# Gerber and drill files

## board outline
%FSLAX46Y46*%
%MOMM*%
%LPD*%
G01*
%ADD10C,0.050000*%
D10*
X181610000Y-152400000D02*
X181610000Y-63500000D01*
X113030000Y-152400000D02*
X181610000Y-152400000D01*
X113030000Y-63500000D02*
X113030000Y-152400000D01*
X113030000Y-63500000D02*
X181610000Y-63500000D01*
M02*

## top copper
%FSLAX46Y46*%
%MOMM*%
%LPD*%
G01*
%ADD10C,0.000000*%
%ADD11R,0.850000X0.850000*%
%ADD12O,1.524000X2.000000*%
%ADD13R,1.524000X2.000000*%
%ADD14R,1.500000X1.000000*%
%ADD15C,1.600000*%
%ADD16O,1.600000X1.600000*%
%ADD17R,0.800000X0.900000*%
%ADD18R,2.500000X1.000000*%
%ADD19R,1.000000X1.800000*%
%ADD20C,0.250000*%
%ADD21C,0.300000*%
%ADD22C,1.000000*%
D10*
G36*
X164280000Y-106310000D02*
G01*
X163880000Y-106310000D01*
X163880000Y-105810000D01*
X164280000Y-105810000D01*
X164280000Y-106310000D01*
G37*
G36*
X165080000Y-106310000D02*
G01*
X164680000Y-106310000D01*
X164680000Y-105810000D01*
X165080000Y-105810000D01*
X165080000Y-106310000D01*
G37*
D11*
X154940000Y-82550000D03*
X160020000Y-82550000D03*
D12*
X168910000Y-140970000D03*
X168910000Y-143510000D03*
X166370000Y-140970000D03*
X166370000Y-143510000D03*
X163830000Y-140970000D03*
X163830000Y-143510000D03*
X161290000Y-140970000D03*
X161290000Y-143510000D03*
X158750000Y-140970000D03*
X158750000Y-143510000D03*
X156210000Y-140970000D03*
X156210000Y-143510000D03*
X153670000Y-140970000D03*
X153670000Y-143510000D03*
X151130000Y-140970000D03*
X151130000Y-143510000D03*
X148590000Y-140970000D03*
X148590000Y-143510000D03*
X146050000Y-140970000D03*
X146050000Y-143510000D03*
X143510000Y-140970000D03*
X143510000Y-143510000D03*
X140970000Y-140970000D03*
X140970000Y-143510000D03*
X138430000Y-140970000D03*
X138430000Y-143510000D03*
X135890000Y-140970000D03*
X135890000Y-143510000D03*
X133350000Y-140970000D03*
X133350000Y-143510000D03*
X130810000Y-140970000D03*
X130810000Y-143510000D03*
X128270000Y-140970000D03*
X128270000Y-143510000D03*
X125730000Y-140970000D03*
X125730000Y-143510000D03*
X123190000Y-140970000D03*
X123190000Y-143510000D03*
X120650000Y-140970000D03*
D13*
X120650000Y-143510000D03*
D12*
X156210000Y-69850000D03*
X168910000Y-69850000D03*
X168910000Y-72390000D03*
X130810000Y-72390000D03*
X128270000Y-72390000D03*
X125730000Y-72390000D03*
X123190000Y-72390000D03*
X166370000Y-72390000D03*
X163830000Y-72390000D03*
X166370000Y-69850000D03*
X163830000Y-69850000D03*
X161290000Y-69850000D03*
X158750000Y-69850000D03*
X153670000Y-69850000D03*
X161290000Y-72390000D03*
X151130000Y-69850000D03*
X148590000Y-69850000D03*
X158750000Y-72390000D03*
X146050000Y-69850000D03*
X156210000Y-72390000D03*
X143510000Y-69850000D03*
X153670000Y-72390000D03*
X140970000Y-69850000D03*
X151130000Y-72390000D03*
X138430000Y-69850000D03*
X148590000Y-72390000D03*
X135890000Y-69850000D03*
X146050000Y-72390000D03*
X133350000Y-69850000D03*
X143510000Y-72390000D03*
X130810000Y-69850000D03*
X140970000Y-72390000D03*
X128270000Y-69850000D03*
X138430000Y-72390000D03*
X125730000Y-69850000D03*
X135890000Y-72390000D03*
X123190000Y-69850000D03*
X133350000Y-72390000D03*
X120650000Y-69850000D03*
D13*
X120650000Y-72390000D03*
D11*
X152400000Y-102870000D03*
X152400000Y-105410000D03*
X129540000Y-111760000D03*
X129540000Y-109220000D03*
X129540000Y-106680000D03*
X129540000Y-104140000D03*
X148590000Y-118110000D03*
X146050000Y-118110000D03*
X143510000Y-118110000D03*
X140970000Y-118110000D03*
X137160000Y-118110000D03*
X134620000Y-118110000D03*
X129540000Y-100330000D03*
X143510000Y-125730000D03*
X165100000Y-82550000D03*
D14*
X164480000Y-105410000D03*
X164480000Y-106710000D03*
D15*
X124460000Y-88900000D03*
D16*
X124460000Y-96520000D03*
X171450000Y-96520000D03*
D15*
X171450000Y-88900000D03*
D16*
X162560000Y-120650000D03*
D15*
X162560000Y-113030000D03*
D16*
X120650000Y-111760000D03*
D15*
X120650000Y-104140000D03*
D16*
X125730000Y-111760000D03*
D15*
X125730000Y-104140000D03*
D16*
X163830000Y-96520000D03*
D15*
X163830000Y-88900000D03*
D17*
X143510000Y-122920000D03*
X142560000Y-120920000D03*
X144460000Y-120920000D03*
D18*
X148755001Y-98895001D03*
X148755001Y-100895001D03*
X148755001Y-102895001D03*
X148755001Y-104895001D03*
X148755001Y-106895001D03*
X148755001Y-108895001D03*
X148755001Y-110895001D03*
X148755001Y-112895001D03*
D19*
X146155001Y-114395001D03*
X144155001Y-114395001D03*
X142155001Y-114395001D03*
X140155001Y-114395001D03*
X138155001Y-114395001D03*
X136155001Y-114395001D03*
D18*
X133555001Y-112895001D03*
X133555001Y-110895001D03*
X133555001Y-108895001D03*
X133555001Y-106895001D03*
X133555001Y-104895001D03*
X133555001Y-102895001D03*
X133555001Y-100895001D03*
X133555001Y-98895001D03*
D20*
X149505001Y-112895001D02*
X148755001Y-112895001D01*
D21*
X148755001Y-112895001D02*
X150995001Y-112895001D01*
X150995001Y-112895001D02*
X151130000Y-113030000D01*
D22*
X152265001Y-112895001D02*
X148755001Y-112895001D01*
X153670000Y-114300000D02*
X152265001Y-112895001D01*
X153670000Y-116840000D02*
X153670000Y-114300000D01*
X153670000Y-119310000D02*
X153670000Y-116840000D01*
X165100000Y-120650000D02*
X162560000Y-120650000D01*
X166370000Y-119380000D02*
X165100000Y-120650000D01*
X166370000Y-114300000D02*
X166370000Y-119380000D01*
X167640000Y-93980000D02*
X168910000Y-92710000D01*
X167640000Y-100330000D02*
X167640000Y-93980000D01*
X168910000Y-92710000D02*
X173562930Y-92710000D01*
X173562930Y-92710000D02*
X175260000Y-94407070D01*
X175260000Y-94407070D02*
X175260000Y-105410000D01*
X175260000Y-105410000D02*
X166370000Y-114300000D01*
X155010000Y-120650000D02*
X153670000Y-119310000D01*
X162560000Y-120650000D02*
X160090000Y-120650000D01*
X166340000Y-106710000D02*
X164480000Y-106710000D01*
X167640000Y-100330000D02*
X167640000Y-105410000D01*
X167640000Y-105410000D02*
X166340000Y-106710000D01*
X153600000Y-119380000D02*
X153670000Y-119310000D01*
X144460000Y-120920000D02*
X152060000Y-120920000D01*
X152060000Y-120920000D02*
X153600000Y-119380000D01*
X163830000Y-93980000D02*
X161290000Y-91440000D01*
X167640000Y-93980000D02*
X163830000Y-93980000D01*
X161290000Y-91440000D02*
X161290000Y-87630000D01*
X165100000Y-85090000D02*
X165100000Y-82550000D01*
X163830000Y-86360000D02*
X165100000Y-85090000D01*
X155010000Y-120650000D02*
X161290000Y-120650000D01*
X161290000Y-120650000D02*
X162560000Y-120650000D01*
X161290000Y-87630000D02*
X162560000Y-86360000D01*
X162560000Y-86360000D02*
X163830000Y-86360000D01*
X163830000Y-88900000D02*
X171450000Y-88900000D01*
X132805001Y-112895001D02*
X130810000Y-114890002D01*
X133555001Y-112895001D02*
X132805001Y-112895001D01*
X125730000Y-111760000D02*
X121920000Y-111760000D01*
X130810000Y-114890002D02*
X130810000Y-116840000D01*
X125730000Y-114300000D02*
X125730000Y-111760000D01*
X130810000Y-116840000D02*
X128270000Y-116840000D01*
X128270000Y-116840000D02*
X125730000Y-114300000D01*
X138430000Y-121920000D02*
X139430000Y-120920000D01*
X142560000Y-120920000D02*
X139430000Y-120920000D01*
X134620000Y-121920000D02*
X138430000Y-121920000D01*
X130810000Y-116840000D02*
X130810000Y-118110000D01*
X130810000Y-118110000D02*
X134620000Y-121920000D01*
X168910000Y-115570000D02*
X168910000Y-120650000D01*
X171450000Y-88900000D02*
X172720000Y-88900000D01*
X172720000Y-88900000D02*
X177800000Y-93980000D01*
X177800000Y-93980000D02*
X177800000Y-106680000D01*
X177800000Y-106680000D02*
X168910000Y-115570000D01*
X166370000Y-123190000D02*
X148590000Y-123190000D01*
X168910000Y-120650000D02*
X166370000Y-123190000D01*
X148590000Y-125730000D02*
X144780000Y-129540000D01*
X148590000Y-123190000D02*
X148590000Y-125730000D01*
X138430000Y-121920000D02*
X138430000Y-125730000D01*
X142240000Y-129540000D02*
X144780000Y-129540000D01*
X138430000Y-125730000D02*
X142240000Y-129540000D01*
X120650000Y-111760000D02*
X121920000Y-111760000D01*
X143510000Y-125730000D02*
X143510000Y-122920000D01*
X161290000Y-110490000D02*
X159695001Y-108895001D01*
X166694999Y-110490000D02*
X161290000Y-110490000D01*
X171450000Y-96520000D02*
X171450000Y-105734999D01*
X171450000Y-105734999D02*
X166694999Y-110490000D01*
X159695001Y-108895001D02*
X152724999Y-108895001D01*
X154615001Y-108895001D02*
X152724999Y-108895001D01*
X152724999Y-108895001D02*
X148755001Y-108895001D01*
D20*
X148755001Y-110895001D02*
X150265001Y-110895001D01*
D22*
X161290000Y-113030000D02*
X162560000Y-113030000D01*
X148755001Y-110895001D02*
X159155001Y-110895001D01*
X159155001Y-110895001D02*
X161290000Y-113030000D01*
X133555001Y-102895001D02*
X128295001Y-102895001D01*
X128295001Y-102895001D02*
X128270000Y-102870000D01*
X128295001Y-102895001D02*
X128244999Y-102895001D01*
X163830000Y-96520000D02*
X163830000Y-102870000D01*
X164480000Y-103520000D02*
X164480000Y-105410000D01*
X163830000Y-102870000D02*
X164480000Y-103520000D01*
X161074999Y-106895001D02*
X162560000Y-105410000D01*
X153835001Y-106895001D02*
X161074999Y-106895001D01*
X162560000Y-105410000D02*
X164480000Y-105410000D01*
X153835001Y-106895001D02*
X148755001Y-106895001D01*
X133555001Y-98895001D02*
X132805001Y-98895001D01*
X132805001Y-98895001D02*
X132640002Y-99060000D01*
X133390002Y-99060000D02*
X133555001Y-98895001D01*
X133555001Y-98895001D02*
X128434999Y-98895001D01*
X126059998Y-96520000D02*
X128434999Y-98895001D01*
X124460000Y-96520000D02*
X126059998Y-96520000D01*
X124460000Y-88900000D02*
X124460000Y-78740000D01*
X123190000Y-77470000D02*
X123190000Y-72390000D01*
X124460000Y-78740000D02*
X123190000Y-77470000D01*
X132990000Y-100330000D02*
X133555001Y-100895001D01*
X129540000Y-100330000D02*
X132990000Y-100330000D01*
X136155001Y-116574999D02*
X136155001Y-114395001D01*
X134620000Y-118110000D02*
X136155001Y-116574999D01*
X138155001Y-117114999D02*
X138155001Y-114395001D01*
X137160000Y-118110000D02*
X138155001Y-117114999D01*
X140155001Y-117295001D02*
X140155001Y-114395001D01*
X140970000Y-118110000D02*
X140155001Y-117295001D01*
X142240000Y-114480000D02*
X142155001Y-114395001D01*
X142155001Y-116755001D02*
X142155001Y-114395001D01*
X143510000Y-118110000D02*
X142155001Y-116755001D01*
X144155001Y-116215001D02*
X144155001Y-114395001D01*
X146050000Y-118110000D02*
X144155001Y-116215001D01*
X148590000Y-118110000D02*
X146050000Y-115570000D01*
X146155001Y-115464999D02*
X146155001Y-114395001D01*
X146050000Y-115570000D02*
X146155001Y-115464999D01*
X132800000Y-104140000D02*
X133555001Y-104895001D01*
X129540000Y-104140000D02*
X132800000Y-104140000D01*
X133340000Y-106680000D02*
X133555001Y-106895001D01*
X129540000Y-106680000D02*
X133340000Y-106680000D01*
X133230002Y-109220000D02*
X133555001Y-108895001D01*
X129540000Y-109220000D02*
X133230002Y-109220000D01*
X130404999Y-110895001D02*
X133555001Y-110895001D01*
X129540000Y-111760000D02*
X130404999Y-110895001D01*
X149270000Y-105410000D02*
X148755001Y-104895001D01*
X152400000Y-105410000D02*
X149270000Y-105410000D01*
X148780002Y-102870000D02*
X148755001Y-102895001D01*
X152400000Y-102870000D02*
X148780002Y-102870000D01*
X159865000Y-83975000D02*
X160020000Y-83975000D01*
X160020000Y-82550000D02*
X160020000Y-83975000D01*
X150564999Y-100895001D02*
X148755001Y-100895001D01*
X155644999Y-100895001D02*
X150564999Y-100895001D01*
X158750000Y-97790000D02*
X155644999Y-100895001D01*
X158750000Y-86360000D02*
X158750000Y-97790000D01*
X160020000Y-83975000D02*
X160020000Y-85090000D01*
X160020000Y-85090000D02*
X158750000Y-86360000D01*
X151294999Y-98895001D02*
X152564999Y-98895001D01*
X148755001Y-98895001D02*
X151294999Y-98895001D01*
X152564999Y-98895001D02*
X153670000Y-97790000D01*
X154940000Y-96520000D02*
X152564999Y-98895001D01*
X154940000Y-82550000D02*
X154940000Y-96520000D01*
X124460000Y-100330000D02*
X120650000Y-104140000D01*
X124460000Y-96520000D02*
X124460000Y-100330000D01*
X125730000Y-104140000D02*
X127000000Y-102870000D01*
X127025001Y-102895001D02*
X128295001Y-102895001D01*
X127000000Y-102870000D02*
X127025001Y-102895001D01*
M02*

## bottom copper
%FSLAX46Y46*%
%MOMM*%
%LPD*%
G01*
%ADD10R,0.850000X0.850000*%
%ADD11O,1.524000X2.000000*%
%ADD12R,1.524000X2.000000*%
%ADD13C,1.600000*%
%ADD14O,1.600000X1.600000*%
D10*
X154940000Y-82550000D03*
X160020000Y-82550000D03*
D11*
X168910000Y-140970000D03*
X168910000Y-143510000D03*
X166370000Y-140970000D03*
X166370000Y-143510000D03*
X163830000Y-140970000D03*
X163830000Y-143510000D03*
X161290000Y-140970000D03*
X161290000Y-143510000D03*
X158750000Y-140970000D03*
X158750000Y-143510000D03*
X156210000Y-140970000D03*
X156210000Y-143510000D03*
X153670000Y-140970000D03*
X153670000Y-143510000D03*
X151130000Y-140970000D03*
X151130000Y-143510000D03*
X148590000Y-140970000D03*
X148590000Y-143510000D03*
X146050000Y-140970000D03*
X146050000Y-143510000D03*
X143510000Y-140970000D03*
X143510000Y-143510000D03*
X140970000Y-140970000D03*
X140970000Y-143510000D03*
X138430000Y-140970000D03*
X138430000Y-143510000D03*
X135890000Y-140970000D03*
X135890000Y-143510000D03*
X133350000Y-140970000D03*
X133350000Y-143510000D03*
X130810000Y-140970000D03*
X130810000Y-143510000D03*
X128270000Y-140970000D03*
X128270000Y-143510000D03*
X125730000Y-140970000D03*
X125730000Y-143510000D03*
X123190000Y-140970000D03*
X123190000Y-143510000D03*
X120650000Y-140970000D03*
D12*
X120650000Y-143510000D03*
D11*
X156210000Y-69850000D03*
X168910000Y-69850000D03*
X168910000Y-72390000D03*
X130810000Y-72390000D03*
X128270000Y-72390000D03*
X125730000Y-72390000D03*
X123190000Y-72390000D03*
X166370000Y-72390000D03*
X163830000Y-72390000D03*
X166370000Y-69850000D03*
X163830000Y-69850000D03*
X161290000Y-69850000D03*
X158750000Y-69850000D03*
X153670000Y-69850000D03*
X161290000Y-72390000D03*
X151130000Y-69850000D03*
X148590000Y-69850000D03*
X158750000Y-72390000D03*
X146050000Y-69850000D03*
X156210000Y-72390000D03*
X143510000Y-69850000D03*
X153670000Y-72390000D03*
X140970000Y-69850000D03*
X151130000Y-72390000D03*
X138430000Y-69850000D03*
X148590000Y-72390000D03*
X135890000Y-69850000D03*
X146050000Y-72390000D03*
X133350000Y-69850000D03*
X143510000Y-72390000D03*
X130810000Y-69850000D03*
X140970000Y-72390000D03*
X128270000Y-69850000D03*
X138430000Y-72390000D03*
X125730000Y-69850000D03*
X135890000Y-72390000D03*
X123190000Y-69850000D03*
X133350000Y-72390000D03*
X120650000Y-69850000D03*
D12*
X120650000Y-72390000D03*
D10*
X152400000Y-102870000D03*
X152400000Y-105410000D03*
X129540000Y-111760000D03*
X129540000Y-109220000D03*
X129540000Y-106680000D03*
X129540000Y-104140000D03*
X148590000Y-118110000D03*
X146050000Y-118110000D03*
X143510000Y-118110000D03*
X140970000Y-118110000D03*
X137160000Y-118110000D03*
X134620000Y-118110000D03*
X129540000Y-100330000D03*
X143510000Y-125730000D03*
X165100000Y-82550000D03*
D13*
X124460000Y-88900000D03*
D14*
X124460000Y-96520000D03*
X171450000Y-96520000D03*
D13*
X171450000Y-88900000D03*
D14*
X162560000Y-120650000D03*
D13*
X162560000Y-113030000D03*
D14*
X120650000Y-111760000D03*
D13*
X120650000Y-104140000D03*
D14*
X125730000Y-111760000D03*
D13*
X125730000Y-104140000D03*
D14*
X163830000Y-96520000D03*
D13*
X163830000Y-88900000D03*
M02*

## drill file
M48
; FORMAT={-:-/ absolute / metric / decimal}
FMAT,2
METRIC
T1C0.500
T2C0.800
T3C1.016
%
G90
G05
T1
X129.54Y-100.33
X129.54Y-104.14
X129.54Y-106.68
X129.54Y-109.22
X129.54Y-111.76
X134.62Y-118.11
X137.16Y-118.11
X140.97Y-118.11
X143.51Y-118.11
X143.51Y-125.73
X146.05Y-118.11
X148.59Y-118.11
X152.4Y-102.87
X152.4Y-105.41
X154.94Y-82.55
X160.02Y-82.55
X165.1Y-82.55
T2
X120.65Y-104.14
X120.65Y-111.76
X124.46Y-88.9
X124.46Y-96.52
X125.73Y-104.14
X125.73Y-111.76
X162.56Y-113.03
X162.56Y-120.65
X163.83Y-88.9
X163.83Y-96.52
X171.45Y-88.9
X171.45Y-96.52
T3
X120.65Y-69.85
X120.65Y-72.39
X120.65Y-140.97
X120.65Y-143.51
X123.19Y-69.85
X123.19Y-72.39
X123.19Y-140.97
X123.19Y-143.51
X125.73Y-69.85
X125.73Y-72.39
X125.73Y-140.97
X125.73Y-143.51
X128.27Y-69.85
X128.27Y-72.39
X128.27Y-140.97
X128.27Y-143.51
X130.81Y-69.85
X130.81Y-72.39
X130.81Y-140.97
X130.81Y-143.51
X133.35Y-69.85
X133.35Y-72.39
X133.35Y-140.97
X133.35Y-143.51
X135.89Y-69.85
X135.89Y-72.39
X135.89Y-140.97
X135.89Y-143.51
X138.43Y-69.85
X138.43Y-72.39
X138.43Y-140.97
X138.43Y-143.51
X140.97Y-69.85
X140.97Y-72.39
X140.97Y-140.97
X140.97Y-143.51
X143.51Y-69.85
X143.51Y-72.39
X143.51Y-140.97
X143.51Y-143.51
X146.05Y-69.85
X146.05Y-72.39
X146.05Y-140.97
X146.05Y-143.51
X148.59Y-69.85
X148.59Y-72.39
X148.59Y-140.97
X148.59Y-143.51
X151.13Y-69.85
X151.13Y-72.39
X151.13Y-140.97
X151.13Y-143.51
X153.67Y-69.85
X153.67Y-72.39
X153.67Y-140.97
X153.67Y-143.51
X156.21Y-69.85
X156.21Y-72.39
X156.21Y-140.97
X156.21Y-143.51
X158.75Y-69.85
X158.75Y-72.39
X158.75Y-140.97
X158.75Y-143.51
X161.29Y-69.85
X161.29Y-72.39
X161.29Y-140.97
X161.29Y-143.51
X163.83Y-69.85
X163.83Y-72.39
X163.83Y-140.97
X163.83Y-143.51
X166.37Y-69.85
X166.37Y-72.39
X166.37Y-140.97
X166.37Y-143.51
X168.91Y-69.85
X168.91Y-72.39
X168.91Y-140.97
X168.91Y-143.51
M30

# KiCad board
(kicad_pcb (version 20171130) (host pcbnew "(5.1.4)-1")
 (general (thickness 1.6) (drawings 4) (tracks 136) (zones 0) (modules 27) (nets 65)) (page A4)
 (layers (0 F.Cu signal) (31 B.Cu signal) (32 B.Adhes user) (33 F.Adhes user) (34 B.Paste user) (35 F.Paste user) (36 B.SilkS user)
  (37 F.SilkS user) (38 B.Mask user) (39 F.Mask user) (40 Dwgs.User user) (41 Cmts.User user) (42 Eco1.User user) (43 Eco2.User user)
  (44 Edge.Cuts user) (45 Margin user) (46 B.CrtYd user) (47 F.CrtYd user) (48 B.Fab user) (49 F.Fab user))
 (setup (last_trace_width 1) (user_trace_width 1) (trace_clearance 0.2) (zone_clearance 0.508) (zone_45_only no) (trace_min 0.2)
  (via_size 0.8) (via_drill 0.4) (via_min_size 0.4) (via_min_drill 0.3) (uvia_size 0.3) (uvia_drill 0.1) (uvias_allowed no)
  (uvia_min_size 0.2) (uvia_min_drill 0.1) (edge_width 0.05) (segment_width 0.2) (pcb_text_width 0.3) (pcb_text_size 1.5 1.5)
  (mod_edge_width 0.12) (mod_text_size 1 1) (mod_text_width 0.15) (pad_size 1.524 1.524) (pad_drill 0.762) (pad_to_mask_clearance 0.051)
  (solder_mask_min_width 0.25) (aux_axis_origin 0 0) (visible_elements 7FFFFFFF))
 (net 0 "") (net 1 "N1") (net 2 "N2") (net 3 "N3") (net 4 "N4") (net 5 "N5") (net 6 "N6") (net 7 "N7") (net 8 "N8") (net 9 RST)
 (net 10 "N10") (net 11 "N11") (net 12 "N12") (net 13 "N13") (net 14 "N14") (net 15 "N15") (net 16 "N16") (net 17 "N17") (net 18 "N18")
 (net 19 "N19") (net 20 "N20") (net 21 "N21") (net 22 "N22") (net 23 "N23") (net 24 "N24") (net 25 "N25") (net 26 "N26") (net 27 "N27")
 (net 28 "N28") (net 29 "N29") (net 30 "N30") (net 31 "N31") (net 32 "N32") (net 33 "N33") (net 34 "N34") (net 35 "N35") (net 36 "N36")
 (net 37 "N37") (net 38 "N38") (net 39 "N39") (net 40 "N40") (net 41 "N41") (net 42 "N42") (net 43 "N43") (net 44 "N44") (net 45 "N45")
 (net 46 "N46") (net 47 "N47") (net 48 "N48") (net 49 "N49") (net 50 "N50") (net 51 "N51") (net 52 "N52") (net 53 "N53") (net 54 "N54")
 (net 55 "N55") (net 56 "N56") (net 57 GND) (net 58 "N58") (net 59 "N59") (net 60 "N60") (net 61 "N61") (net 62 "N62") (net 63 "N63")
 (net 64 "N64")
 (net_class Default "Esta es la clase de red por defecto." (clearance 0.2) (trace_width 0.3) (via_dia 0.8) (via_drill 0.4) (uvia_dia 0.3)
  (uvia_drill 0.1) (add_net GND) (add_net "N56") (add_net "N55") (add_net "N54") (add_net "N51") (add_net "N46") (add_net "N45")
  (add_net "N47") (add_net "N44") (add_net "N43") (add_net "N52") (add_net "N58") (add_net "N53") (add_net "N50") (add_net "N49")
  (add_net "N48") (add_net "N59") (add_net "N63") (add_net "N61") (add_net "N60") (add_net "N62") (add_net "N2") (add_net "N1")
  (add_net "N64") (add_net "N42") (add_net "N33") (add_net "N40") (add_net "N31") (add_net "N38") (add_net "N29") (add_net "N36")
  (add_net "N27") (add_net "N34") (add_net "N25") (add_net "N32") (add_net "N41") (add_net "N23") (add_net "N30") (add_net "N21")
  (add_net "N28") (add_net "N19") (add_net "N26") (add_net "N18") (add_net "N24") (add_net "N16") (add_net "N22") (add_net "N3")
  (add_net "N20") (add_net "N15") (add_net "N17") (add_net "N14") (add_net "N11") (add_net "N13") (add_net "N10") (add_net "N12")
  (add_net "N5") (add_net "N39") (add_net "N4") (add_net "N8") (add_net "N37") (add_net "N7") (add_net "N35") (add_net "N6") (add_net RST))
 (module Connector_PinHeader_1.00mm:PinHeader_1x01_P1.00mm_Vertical (layer F.Cu) (at 154.94 82.55)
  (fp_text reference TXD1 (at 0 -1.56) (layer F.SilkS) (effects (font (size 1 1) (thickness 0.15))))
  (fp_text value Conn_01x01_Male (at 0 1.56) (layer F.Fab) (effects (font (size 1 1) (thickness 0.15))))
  (pad 1 thru_hole rect (at 0 0) (size 0.85 0.85) (drill 0.5) (layers *.Cu *.Mask) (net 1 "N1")))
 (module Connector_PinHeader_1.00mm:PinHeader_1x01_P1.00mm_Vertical (layer F.Cu) (at 160.02 82.55)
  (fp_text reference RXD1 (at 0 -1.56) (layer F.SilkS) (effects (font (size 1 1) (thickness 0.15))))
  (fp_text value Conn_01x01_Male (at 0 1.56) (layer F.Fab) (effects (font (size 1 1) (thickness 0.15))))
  (pad 1 thru_hole rect (at 0 0) (size 0.85 0.85) (drill 0.5) (layers *.Cu *.Mask) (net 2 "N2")))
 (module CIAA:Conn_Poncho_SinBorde (layer F.Cu) (at 120.65 72.39 90)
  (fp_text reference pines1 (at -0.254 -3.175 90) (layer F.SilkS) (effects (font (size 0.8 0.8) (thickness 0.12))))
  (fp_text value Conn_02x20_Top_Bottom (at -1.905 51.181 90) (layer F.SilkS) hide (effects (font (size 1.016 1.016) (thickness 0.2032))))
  (pad 80 thru_hole oval (at -68.58 48.26) (size 1.524 2) (drill 1.016) (layers *.Cu *.Mask F.SilkS))
  (pad 79 thru_hole oval (at -71.12 48.26) (size 1.524 2) (drill 1.016) (layers *.Cu *.Mask F.SilkS))
  (pad 78 thru_hole oval (at -68.58 45.72) (size 1.524 2) (drill 1.016) (layers *.Cu *.Mask F.SilkS))
  (pad 77 thru_hole oval (at -71.12 45.72) (size 1.524 2) (drill 1.016) (layers *.Cu *.Mask F.SilkS))
  (pad 76 thru_hole oval (at -68.58 43.18) (size 1.524 2) (drill 1.016) (layers *.Cu *.Mask F.SilkS))
  (pad 75 thru_hole oval (at -71.12 43.18) (size 1.524 2) (drill 1.016) (layers *.Cu *.Mask F.SilkS))
  (pad 74 thru_hole oval (at -68.58 40.64) (size 1.524 2) (drill 1.016) (layers *.Cu *.Mask F.SilkS))
  (pad 73 thru_hole oval (at -71.12 40.64) (size 1.524 2) (drill 1.016) (layers *.Cu *.Mask F.SilkS))
  (pad 72 thru_hole oval (at -68.58 38.1) (size 1.524 2) (drill 1.016) (layers *.Cu *.Mask F.SilkS))
  (pad 71 thru_hole oval (at -71.12 38.1) (size 1.524 2) (drill 1.016) (layers *.Cu *.Mask F.SilkS))
  (pad 70 thru_hole oval (at -68.58 35.56) (size 1.524 2) (drill 1.016) (layers *.Cu *.Mask F.SilkS))
  (pad 69 thru_hole oval (at -71.12 35.56) (size 1.524 2) (drill 1.016) (layers *.Cu *.Mask F.SilkS))
  (pad 68 thru_hole oval (at -68.58 33.02) (size 1.524 2) (drill 1.016) (layers *.Cu *.Mask F.SilkS))
  (pad 67 thru_hole oval (at -71.12 33.02) (size 1.524 2) (drill 1.016) (layers *.Cu *.Mask F.SilkS))
  (pad 66 thru_hole oval (at -68.58 30.48) (size 1.524 2) (drill 1.016) (layers *.Cu *.Mask F.SilkS))
  (pad 65 thru_hole oval (at -71.12 30.48) (size 1.524 2) (drill 1.016) (layers *.Cu *.Mask F.SilkS))
  (pad 64 thru_hole oval (at -68.58 27.94) (size 1.524 2) (drill 1.016) (layers *.Cu *.Mask F.SilkS))
  (pad 63 thru_hole oval (at -71.12 27.94) (size 1.524 2) (drill 1.016) (layers *.Cu *.Mask F.SilkS))
  (pad 62 thru_hole oval (at -68.58 25.4) (size 1.524 2) (drill 1.016) (layers *.Cu *.Mask F.SilkS))
  (pad 61 thru_hole oval (at -71.12 25.4) (size 1.524 2) (drill 1.016) (layers *.Cu *.Mask F.SilkS))
  (pad 60 thru_hole oval (at -68.58 22.86) (size 1.524 2) (drill 1.016) (layers *.Cu *.Mask F.SilkS))
  (pad 59 thru_hole oval (at -71.12 22.86) (size 1.524 2) (drill 1.016) (layers *.Cu *.Mask F.SilkS))
  (pad 58 thru_hole oval (at -68.58 20.32) (size 1.524 2) (drill 1.016) (layers *.Cu *.Mask F.SilkS))
  (pad 57 thru_hole oval (at -71.12 20.32) (size 1.524 2) (drill 1.016) (layers *.Cu *.Mask F.SilkS))
  (pad 56 thru_hole oval (at -68.58 17.78) (size 1.524 2) (drill 1.016) (layers *.Cu *.Mask F.SilkS))
  (pad 55 thru_hole oval (at -71.12 17.78) (size 1.524 2) (drill 1.016) (layers *.Cu *.Mask F.SilkS))
  (pad 54 thru_hole oval (at -68.58 15.24) (size 1.524 2) (drill 1.016) (layers *.Cu *.Mask F.SilkS))
  (pad 53 thru_hole oval (at -71.12 15.24) (size 1.524 2) (drill 1.016) (layers *.Cu *.Mask F.SilkS))
  (pad 52 thru_hole oval (at -68.58 12.7) (size 1.524 2) (drill 1.016) (layers *.Cu *.Mask F.SilkS))
  (pad 51 thru_hole oval (at -71.12 12.7) (size 1.524 2) (drill 1.016) (layers *.Cu *.Mask F.SilkS))
  (pad 50 thru_hole oval (at -68.58 10.16) (size 1.524 2) (drill 1.016) (layers *.Cu *.Mask F.SilkS))
  (pad 49 thru_hole oval (at -71.12 10.16) (size 1.524 2) (drill 1.016) (layers *.Cu *.Mask F.SilkS))
  (pad 48 thru_hole oval (at -68.58 7.62) (size 1.524 2) (drill 1.016) (layers *.Cu *.Mask F.SilkS))
  (pad 47 thru_hole oval (at -71.12 7.62) (size 1.524 2) (drill 1.016) (layers *.Cu *.Mask F.SilkS))
  (pad 46 thru_hole oval (at -68.58 5.08) (size 1.524 2) (drill 1.016) (layers *.Cu *.Mask F.SilkS))
  (pad 45 thru_hole oval (at -71.12 5.08) (size 1.524 2) (drill 1.016) (layers *.Cu *.Mask F.SilkS))
  (pad 44 thru_hole oval (at -68.58 2.54) (size 1.524 2) (drill 1.016) (layers *.Cu *.Mask F.SilkS))
  (pad 43 thru_hole oval (at -71.12 2.54) (size 1.524 2) (drill 1.016) (layers *.Cu *.Mask F.SilkS))
  (pad 42 thru_hole oval (at -68.58 0) (size 1.524 2) (drill 1.016) (layers *.Cu *.Mask F.SilkS))
  (pad 41 thru_hole rect (at -71.12 0) (size 1.524 2) (drill 1.016) (layers *.Cu *.Mask F.SilkS))
  (pad 30 thru_hole oval (at 2.54 35.56) (size 1.524 2) (drill 1.016) (layers *.Cu *.Mask F.SilkS) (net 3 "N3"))
  (pad 40 thru_hole oval (at 2.54 48.26) (size 1.524 2) (drill 1.016) (layers *.Cu *.Mask F.SilkS) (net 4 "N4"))
  (pad 39 thru_hole oval (at 0 48.26) (size 1.524 2) (drill 1.016) (layers *.Cu *.Mask F.SilkS) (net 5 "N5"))
  (pad 9 thru_hole oval (at 0 10.16) (size 1.524 2) (drill 1.016) (layers *.Cu *.Mask F.SilkS) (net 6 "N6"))
  (pad 7 thru_hole oval (at 0 7.62) (size 1.524 2) (drill 1.016) (layers *.Cu *.Mask F.SilkS) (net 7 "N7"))
  (pad 5 thru_hole oval (at 0 5.08) (size 1.524 2) (drill 1.016) (layers *.Cu *.Mask F.SilkS) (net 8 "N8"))
  (pad 3 thru_hole oval (at 0 2.54) (size 1.524 2) (drill 1.016) (layers *.Cu *.Mask F.SilkS) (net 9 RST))
  (pad 37 thru_hole oval (at 0 45.72) (size 1.524 2) (drill 1.016) (layers *.Cu *.Mask F.SilkS) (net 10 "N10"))
  (pad 35 thru_hole oval (at 0 43.18) (size 1.524 2) (drill 1.016) (layers *.Cu *.Mask F.SilkS) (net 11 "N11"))
  (pad 38 thru_hole oval (at 2.54 45.72) (size 1.524 2) (drill 1.016) (layers *.Cu *.Mask F.SilkS) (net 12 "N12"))
  (pad 36 thru_hole oval (at 2.54 43.18) (size 1.524 2) (drill 1.016) (layers *.Cu *.Mask F.SilkS) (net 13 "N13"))
  (pad 34 thru_hole oval (at 2.54 40.64) (size 1.524 2) (drill 1.016) (layers *.Cu *.Mask F.SilkS) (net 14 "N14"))
  (pad 32 thru_hole oval (at 2.54 38.1) (size 1.524 2) (drill 1.016) (layers *.Cu *.Mask F.SilkS) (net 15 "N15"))
  (pad 28 thru_hole oval (at 2.54 33.02) (size 1.524 2) (drill 1.016) (layers *.Cu *.Mask F.SilkS) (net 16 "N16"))
  (pad 33 thru_hole oval (at 0 40.64) (size 1.524 2) (drill 1.016) (layers *.Cu *.Mask F.SilkS) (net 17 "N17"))
  (pad 26 thru_hole oval (at 2.54 30.48) (size 1.524 2) (drill 1.016) (layers *.Cu *.Mask F.SilkS) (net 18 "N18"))
  (pad 24 thru_hole oval (at 2.54 27.94) (size 1.524 2) (drill 1.016) (layers *.Cu *.Mask F.SilkS) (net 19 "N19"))
  (pad 31 thru_hole oval (at 0 38.1) (size 1.524 2) (drill 1.016) (layers *.Cu *.Mask F.SilkS) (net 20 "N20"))
  (pad 22 thru_hole oval (at 2.54 25.4) (size 1.524 2) (drill 1.016) (layers *.Cu *.Mask F.SilkS) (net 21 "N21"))
  (pad 29 thru_hole oval (at 0 35.56) (size 1.524 2) (drill 1.016) (layers *.Cu *.Mask F.SilkS) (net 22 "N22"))
  (pad 20 thru_hole oval (at 2.54 22.86) (size 1.524 2) (drill 1.016) (layers *.Cu *.Mask F.SilkS) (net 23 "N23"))
  (pad 27 thru_hole oval (at 0 33.02) (size 1.524 2) (drill 1.016) (layers *.Cu *.Mask F.SilkS) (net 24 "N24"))
  (pad 18 thru_hole oval (at 2.54 20.32) (size 1.524 2) (drill 1.016) (layers *.Cu *.Mask F.SilkS) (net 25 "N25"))
  (pad 25 thru_hole oval (at 0 30.48) (size 1.524 2) (drill 1.016) (layers *.Cu *.Mask F.SilkS) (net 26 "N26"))
  (pad 16 thru_hole oval (at 2.54 17.78) (size 1.524 2) (drill 1.016) (layers *.Cu *.Mask F.SilkS) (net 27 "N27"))
  (pad 23 thru_hole oval (at 0 27.94) (size 1.524 2) (drill 1.016) (layers *.Cu *.Mask F.SilkS) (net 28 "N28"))
  (pad 14 thru_hole oval (at 2.54 15.24) (size 1.524 2) (drill 1.016) (layers *.Cu *.Mask F.SilkS) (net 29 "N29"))
  (pad 21 thru_hole oval (at 0 25.4) (size 1.524 2) (drill 1.016) (layers *.Cu *.Mask F.SilkS) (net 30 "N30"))
  (pad 12 thru_hole oval (at 2.54 12.7) (size 1.524 2) (drill 1.016) (layers *.Cu *.Mask F.SilkS) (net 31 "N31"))
  (pad 19 thru_hole oval (at 0 22.86) (size 1.524 2) (drill 1.016) (layers *.Cu *.Mask F.SilkS) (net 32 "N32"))
  (pad 10 thru_hole oval (at 2.54 10.16) (size 1.524 2) (drill 1.016) (layers *.Cu *.Mask F.SilkS) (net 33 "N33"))
  (pad 17 thru_hole oval (at 0 20.32) (size 1.524 2) (drill 1.016) (layers *.Cu *.Mask F.SilkS) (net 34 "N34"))
  (pad 8 thru_hole oval (at 2.54 7.62) (size 1.524 2) (drill 1.016) (layers *.Cu *.Mask F.SilkS) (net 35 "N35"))
  (pad 15 thru_hole oval (at 0 17.78) (size 1.524 2) (drill 1.016) (layers *.Cu *.Mask F.SilkS) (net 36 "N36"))
  (pad 6 thru_hole oval (at 2.54 5.08) (size 1.524 2) (drill 1.016) (layers *.Cu *.Mask F.SilkS) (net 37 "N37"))
  (pad 13 thru_hole oval (at 0 15.24) (size 1.524 2) (drill 1.016) (layers *.Cu *.Mask F.SilkS) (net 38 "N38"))
  (pad 4 thru_hole oval (at 2.54 2.54) (size 1.524 2) (drill 1.016) (layers *.Cu *.Mask F.SilkS) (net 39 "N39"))
  (pad 11 thru_hole oval (at 0 12.7) (size 1.524 2) (drill 1.016) (layers *.Cu *.Mask F.SilkS) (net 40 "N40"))
  (pad 2 thru_hole oval (at 2.54 0) (size 1.524 2) (drill 1.016) (layers *.Cu *.Mask F.SilkS) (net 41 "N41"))
  (pad 1 thru_hole rect (at 0 0) (size 1.524 2) (drill 1.016) (layers *.Cu *.Mask F.SilkS) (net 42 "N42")))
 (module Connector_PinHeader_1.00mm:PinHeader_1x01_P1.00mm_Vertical (layer F.Cu) (at 152.4 102.87)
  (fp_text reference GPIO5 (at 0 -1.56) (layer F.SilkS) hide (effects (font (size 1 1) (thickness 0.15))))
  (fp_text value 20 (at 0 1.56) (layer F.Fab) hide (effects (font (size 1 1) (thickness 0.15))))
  (pad 1 thru_hole rect (at 0 0) (size 0.85 0.85) (drill 0.5) (layers *.Cu *.Mask) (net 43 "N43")))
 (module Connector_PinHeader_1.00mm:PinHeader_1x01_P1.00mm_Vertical (layer F.Cu) (at 152.4 105.41)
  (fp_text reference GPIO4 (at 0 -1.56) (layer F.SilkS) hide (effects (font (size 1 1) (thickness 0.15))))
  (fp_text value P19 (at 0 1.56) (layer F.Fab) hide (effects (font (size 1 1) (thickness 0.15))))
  (pad 1 thru_hole rect (at 0 0) (size 0.85 0.85) (drill 0.5) (layers *.Cu *.Mask) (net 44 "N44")))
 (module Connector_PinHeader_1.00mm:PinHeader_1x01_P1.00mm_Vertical (layer F.Cu) (at 129.54 111.76)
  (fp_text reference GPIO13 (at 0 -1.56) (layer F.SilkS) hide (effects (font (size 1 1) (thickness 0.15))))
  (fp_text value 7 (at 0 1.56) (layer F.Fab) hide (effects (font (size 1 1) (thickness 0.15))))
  (pad 1 thru_hole rect (at 0 0) (size 0.85 0.85) (drill 0.5) (layers *.Cu *.Mask) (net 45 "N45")))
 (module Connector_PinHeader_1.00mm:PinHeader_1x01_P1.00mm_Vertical (layer F.Cu) (at 129.54 109.22)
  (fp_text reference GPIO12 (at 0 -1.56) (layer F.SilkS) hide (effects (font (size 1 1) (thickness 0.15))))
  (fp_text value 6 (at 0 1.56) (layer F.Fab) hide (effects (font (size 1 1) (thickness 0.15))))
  (pad 1 thru_hole rect (at 0 0) (size 0.85 0.85) (drill 0.5) (layers *.Cu *.Mask) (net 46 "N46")))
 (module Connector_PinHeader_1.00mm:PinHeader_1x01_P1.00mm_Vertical (layer F.Cu) (at 129.54 106.68)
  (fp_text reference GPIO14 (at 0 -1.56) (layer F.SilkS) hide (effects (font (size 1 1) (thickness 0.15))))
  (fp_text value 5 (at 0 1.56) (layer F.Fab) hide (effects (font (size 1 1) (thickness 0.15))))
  (pad 1 thru_hole rect (at 0 0) (size 0.85 0.85) (drill 0.5) (layers *.Cu *.Mask) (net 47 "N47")))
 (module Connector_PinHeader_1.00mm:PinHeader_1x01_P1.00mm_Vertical (layer F.Cu) (at 129.54 104.14)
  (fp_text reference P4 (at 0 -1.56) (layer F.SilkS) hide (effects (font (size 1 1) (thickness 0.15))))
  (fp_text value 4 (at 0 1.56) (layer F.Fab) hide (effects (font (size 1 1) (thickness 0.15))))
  (pad 1 thru_hole rect (at 0 0) (size 0.85 0.85) (drill 0.5) (layers *.Cu *.Mask) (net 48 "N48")))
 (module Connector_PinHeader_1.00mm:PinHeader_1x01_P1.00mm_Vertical (layer F.Cu) (at 148.59 118.11)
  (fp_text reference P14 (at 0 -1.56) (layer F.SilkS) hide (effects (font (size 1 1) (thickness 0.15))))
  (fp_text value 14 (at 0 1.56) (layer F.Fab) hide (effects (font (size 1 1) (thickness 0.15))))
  (pad 1 thru_hole rect (at 0 0) (size 0.85 0.85) (drill 0.5) (layers *.Cu *.Mask) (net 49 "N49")))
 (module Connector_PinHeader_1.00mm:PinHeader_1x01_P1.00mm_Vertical (layer F.Cu) (at 146.05 118.11)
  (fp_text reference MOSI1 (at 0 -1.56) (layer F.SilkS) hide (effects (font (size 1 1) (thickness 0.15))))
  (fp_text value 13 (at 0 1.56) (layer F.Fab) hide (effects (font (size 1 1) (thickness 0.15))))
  (pad 1 thru_hole rect (at 0 0) (size 0.85 0.85) (drill 0.5) (layers *.Cu *.Mask) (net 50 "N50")))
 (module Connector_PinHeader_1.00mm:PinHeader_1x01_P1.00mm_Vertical (layer F.Cu) (at 143.51 118.11)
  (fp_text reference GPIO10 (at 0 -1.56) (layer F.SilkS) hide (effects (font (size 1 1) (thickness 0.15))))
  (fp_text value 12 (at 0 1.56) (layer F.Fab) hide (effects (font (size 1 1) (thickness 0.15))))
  (pad 1 thru_hole rect (at 0 0) (size 0.85 0.85) (drill 0.5) (layers *.Cu *.Mask) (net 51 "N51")))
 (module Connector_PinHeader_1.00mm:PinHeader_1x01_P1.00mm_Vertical (layer F.Cu) (at 140.97 118.11)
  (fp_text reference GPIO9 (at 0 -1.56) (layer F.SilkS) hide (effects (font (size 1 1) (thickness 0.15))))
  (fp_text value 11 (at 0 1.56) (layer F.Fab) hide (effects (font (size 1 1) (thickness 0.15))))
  (pad 1 thru_hole rect (at 0 0) (size 0.85 0.85) (drill 0.5) (layers *.Cu *.Mask) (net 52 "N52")))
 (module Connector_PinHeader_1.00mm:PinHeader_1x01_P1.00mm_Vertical (layer F.Cu) (at 137.16 118.11)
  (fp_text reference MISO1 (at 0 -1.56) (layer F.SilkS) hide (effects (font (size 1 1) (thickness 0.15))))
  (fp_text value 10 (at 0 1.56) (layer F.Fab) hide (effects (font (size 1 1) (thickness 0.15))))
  (pad 1 thru_hole rect (at 0 0) (size 0.85 0.85) (drill 0.5) (layers *.Cu *.Mask) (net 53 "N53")))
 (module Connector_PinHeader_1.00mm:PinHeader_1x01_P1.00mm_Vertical (layer F.Cu) (at 134.62 118.11)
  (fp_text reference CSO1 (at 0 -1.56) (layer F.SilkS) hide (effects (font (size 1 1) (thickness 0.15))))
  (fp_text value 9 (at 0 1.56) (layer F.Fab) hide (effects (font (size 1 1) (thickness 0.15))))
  (pad 1 thru_hole rect (at 0 0) (size 0.85 0.85) (drill 0.5) (layers *.Cu *.Mask) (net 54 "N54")))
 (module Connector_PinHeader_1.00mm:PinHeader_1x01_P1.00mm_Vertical (layer F.Cu) (at 129.54 100.33)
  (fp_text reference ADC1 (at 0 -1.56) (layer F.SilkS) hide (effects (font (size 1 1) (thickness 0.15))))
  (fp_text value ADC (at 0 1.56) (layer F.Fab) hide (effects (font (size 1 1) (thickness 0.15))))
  (pad 1 thru_hole rect (at 0 0) (size 0.85 0.85) (drill 0.5) (layers *.Cu *.Mask) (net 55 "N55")))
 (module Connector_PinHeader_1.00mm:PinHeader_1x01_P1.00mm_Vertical (layer F.Cu) (at 143.51 125.73 180)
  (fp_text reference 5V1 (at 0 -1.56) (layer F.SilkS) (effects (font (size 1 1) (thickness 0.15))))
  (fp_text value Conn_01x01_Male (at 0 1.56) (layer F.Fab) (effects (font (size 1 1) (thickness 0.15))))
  (pad 1 thru_hole rect (at 0 0 180) (size 0.85 0.85) (drill 0.5) (layers *.Cu *.Mask) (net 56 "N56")))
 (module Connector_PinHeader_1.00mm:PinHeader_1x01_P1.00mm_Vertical (layer F.Cu) (at 165.1 82.55)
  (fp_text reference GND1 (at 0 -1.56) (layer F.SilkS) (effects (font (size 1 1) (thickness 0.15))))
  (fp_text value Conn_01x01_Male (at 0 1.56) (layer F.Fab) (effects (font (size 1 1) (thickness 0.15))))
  (pad 1 thru_hole rect (at 0 0) (size 0.85 0.85) (drill 0.5) (layers *.Cu *.Mask) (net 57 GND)))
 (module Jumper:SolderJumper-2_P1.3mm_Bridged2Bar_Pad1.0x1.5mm (layer F.Cu) (at 164.48 106.06 90)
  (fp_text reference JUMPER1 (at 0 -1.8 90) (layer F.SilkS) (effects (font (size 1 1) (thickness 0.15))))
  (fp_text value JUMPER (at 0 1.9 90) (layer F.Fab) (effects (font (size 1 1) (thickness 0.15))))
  (fp_poly (pts (xy -0.25 -0.6) (xy 0.25 -0.6) (xy 0.25 -0.2) (xy -0.25 -0.2)) (layer F.Cu) (width 0))
  (fp_poly (pts (xy -0.25 0.2) (xy 0.25 0.2) (xy 0.25 0.6) (xy -0.25 0.6)) (layer F.Cu) (width 0))
  (pad 2 smd rect (at 0.65 0 90) (size 1 1.5) (layers F.Cu F.Mask) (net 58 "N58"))
  (pad 1 smd rect (at -0.65 0 90) (size 1 1.5) (layers F.Cu F.Mask) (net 57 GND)))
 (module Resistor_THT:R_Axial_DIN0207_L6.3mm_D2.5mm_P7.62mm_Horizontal (layer F.Cu) (at 124.46 88.9 270)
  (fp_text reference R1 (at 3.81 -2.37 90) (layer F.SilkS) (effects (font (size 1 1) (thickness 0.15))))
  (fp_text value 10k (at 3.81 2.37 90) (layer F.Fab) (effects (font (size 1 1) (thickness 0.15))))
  (pad 1 thru_hole circle (at 0 0 270) (size 1.6 1.6) (drill 0.8) (layers *.Cu *.Mask) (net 9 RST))
  (pad 2 thru_hole oval (at 7.62 0 270) (size 1.6 1.6) (drill 0.8) (layers *.Cu *.Mask) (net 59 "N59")))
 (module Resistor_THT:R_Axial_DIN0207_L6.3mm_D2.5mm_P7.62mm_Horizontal (layer F.Cu) (at 171.45 88.9 270)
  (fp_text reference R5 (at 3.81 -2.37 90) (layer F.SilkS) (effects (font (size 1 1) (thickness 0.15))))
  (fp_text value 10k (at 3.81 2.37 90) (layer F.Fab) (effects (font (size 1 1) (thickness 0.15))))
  (pad 2 thru_hole oval (at 7.62 0 270) (size 1.6 1.6) (drill 0.8) (layers *.Cu *.Mask) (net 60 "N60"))
  (pad 1 thru_hole circle (at 0 0 270) (size 1.6 1.6) (drill 0.8) (layers *.Cu *.Mask) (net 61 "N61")))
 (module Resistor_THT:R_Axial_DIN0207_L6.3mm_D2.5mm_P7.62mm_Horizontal (layer F.Cu) (at 162.56 113.03 270)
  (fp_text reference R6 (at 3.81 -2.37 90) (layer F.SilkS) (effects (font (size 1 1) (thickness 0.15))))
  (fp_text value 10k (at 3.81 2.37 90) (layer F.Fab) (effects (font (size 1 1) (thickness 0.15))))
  (pad 2 thru_hole oval (at 7.62 0 270) (size 1.6 1.6) (drill 0.8) (layers *.Cu *.Mask) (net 57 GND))
  (pad 1 thru_hole circle (at 0 0 270) (size 1.6 1.6) (drill 0.8) (layers *.Cu *.Mask) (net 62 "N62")))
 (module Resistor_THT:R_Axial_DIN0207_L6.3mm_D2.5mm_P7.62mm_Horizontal (layer F.Cu) (at 120.65 104.14 270)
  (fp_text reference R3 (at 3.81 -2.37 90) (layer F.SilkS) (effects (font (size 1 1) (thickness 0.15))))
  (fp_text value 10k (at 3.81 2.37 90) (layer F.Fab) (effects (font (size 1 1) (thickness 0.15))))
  (pad 2 thru_hole oval (at 7.62 0 270) (size 1.6 1.6) (drill 0.8) (layers *.Cu *.Mask) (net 61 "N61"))
  (pad 1 thru_hole circle (at 0 0 270) (size 1.6 1.6) (drill 0.8) (layers *.Cu *.Mask) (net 59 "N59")))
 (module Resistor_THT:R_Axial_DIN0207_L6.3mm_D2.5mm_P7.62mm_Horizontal (layer F.Cu) (at 125.73 104.14 270)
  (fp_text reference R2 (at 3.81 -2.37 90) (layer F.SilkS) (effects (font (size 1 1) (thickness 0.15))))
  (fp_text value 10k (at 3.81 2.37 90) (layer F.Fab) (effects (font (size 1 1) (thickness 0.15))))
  (pad 2 thru_hole oval (at 7.62 0 270) (size 1.6 1.6) (drill 0.8) (layers *.Cu *.Mask) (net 61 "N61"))
  (pad 1 thru_hole circle (at 0 0 270) (size 1.6 1.6) (drill 0.8) (layers *.Cu *.Mask) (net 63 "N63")))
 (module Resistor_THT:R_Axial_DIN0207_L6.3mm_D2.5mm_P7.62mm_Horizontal (layer F.Cu) (at 163.83 88.9 270)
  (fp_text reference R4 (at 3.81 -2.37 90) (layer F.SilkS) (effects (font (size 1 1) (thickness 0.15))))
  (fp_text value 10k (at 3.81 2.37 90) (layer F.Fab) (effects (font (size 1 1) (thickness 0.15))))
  (pad 2 thru_hole oval (at 7.62 0 270) (size 1.6 1.6) (drill 0.8) (layers *.Cu *.Mask) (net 58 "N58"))
  (pad 1 thru_hole circle (at 0 0 270) (size 1.6 1.6) (drill 0.8) (layers *.Cu *.Mask) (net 61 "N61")))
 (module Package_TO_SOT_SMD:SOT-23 (layer F.Cu) (at 143.51 121.92 270)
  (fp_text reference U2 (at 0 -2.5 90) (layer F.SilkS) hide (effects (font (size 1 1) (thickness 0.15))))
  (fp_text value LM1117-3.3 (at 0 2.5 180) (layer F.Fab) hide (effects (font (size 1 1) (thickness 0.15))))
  (pad 3 smd rect (at 1 0 270) (size 0.9 0.8) (layers F.Cu F.Paste F.Mask) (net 56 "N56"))
  (pad 2 smd rect (at -1 0.95 270) (size 0.9 0.8) (layers F.Cu F.Paste F.Mask) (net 61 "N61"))
  (pad 1 smd rect (at -1 -0.95 270) (size 0.9 0.8) (layers F.Cu F.Paste F.Mask) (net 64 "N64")))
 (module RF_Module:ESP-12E (layer F.Cu) (at 141.155001 102.395001)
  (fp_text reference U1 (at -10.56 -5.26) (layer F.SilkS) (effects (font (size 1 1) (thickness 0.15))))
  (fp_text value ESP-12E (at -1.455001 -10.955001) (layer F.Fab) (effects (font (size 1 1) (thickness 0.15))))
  (pad 22 smd rect (at 7.6 -3.5) (size 2.5 1) (layers F.Cu F.Paste F.Mask) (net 1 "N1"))
  (pad 21 smd rect (at 7.6 -1.5) (size 2.5 1) (layers F.Cu F.Paste F.Mask) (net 2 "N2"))
  (pad 20 smd rect (at 7.6 0.5) (size 2.5 1) (layers F.Cu F.Paste F.Mask) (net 43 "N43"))
  (pad 19 smd rect (at 7.6 2.5) (size 2.5 1) (layers F.Cu F.Paste F.Mask) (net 44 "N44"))
  (pad 18 smd rect (at 7.6 4.5) (size 2.5 1) (layers F.Cu F.Paste F.Mask) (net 58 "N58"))
  (pad 17 smd rect (at 7.6 6.5) (size 2.5 1) (layers F.Cu F.Paste F.Mask) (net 60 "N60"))
  (pad 16 smd rect (at 7.6 8.5) (size 2.5 1) (layers F.Cu F.Paste F.Mask) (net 62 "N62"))
  (pad 15 smd rect (at 7.6 10.5) (size 2.5 1) (layers F.Cu F.Paste F.Mask) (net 57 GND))
  (pad 14 smd rect (at 5 12) (size 1 1.8) (layers F.Cu F.Paste F.Mask) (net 49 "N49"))
  (pad 13 smd rect (at 3 12) (size 1 1.8) (layers F.Cu F.Paste F.Mask) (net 50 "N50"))
  (pad 12 smd rect (at 1 12) (size 1 1.8) (layers F.Cu F.Paste F.Mask) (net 51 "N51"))
  (pad 11 smd rect (at -1 12) (size 1 1.8) (layers F.Cu F.Paste F.Mask) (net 52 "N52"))
  (pad 10 smd rect (at -3 12) (size 1 1.8) (layers F.Cu F.Paste F.Mask) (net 53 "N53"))
  (pad 9 smd rect (at -5 12) (size 1 1.8) (layers F.Cu F.Paste F.Mask) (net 54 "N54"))
  (pad 8 smd rect (at -7.6 10.5) (size 2.5 1) (layers F.Cu F.Paste F.Mask) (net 61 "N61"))
  (pad 7 smd rect (at -7.6 8.5) (size 2.5 1) (layers F.Cu F.Paste F.Mask) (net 45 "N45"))
  (pad 6 smd rect (at -7.6 6.5) (size 2.5 1) (layers F.Cu F.Paste F.Mask) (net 46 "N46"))
  (pad 5 smd rect (at -7.6 4.5) (size 2.5 1) (layers F.Cu F.Paste F.Mask) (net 47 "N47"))
  (pad 4 smd rect (at -7.6 2.5) (size 2.5 1) (layers F.Cu F.Paste F.Mask) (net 48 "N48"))
  (pad 3 smd rect (at -7.6 0.5) (size 2.5 1) (layers F.Cu F.Paste F.Mask) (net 63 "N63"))
  (pad 2 smd rect (at -7.6 -1.5) (size 2.5 1) (layers F.Cu F.Paste F.Mask) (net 55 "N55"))
  (pad 1 smd rect (at -7.6 -3.5) (size 2.5 1) (layers F.Cu F.Paste F.Mask) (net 59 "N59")))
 (gr_line (start 181.61 152.4) (end 181.61 63.5) (layer Edge.Cuts) (width 0.05))
 (gr_line (start 113.03 152.4) (end 181.61 152.4) (layer Edge.Cuts) (width 0.05))
 (gr_line (start 113.03 63.5) (end 113.03 152.4) (layer Edge.Cuts) (width 0.05))
 (gr_line (start 113.03 63.5) (end 181.61 63.5) (layer Edge.Cuts) (width 0.05))
 (segment (start 149.505001 112.895001) (end 148.755001 112.895001) (width 0.25) (layer F.Cu) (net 57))
 (segment (start 148.755001 112.895001) (end 150.995001 112.895001) (width 0.3) (layer F.Cu) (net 57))
 (segment (start 150.995001 112.895001) (end 151.13 113.03) (width 0.3) (layer F.Cu) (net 57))
 (segment (start 152.265001 112.895001) (end 148.755001 112.895001) (width 1) (layer F.Cu) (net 57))
 (segment (start 153.67 114.3) (end 152.265001 112.895001) (width 1) (layer F.Cu) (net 57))
 (segment (start 153.67 116.84) (end 153.67 114.3) (width 1) (layer F.Cu) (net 57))
 (segment (start 153.67 119.31) (end 153.67 116.84) (width 1) (layer F.Cu) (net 57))
 (segment (start 165.1 120.65) (end 162.56 120.65) (width 1) (layer F.Cu) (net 57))
 (segment (start 166.37 119.38) (end 165.1 120.65) (width 1) (layer F.Cu) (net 57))
 (segment (start 166.37 114.3) (end 166.37 119.38) (width 1) (layer F.Cu) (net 57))
 (segment (start 167.64 93.98) (end 168.91 92.71) (width 1) (layer F.Cu) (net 57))
 (segment (start 167.64 100.33) (end 167.64 93.98) (width 1) (layer F.Cu) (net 57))
 (segment (start 168.91 92.71) (end 173.56293 92.71) (width 1) (layer F.Cu) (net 57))
 (segment (start 173.56293 92.71) (end 175.26 94.40707) (width 1) (layer F.Cu) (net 57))
 (segment (start 175.26 94.40707) (end 175.26 105.41) (width 1) (layer F.Cu) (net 57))
 (segment (start 175.26 105.41) (end 166.37 114.3) (width 1) (layer F.Cu) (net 57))
 (segment (start 155.01 120.65) (end 153.67 119.31) (width 1) (layer F.Cu) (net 57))
 (segment (start 162.56 120.65) (end 160.09 120.65) (width 1) (layer F.Cu) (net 57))
 (segment (start 166.34 106.71) (end 164.48 106.71) (width 1) (layer F.Cu) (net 57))
 (segment (start 167.64 100.33) (end 167.64 105.41) (width 1) (layer F.Cu) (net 57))
 (segment (start 167.64 105.41) (end 166.34 106.71) (width 1) (layer F.Cu) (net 57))
 (segment (start 153.6 119.38) (end 153.67 119.31) (width 1) (layer F.Cu) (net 57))
 (segment (start 144.46 120.92) (end 152.06 120.92) (width 1) (layer F.Cu) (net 57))
 (segment (start 152.06 120.92) (end 153.6 119.38) (width 1) (layer F.Cu) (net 57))
 (segment (start 163.83 93.98) (end 161.29 91.44) (width 1) (layer F.Cu) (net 57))
 (segment (start 167.64 93.98) (end 163.83 93.98) (width 1) (layer F.Cu) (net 57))
 (segment (start 161.29 91.44) (end 161.29 87.63) (width 1) (layer F.Cu) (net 57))
 (segment (start 165.1 85.09) (end 165.1 82.55) (width 1) (layer F.Cu) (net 57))
 (segment (start 163.83 86.36) (end 165.1 85.09) (width 1) (layer F.Cu) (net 57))
 (segment (start 155.01 120.65) (end 161.29 120.65) (width 1) (layer F.Cu) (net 57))
 (segment (start 161.29 120.65) (end 162.56 120.65) (width 1) (layer F.Cu) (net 57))
 (segment (start 161.29 87.63) (end 162.56 86.36) (width 1) (layer F.Cu) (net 57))
 (segment (start 162.56 86.36) (end 163.83 86.36) (width 1) (layer F.Cu) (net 57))
 (segment (start 163.83 88.9) (end 171.45 88.9) (width 1) (layer F.Cu) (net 61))
 (segment (start 132.805001 112.895001) (end 130.81 114.890002) (width 1) (layer F.Cu) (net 61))
 (segment (start 133.555001 112.895001) (end 132.805001 112.895001) (width 1) (layer F.Cu) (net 61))
 (segment (start 125.73 111.76) (end 121.92 111.76) (width 1) (layer F.Cu) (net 61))
 (segment (start 130.81 114.890002) (end 130.81 116.84) (width 1) (layer F.Cu) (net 61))
 (segment (start 125.73 114.3) (end 125.73 111.76) (width 1) (layer F.Cu) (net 61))
 (segment (start 130.81 116.84) (end 128.27 116.84) (width 1) (layer F.Cu) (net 61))
 (segment (start 128.27 116.84) (end 125.73 114.3) (width 1) (layer F.Cu) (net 61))
 (segment (start 138.43 121.92) (end 139.43 120.92) (width 1) (layer F.Cu) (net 61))
 (segment (start 142.56 120.92) (end 139.43 120.92) (width 1) (layer F.Cu) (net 61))
 (segment (start 134.62 121.92) (end 138.43 121.92) (width 1) (layer F.Cu) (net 61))
 (segment (start 130.81 116.84) (end 130.81 118.11) (width 1) (layer F.Cu) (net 61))
 (segment (start 130.81 118.11) (end 134.62 121.92) (width 1) (layer F.Cu) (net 61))
 (segment (start 168.91 115.57) (end 168.91 120.65) (width 1) (layer F.Cu) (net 61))
 (segment (start 171.45 88.9) (end 172.72 88.9) (width 1) (layer F.Cu) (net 61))
 (segment (start 172.72 88.9) (end 177.8 93.98) (width 1) (layer F.Cu) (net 61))
 (segment (start 177.8 93.98) (end 177.8 106.68) (width 1) (layer F.Cu) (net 61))
 (segment (start 177.8 106.68) (end 168.91 115.57) (width 1) (layer F.Cu) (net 61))
 (segment (start 166.37 123.19) (end 148.59 123.19) (width 1) (layer F.Cu) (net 61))
 (segment (start 168.91 120.65) (end 166.37 123.19) (width 1) (layer F.Cu) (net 61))
 (segment (start 148.59 125.73) (end 144.78 129.54) (width 1) (layer F.Cu) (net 61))
 (segment (start 148.59 123.19) (end 148.59 125.73) (width 1) (layer F.Cu) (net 61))
 (segment (start 138.43 121.92) (end 138.43 125.73) (width 1) (layer F.Cu) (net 61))
 (segment (start 142.24 129.54) (end 144.78 129.54) (width 1) (layer F.Cu) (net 61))
 (segment (start 138.43 125.73) (end 142.24 129.54) (width 1) (layer F.Cu) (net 61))
 (segment (start 120.65 111.76) (end 121.92 111.76) (width 1) (layer F.Cu) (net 61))
 (segment (start 143.51 125.73) (end 143.51 122.92) (width 1) (layer F.Cu) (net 56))
 (segment (start 161.29 110.49) (end 159.695001 108.895001) (width 1) (layer F.Cu) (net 60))
 (segment (start 166.694999 110.49) (end 161.29 110.49) (width 1) (layer F.Cu) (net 60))
 (segment (start 171.45 96.52) (end 171.45 105.734999) (width 1) (layer F.Cu) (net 60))
 (segment (start 171.45 105.734999) (end 166.694999 110.49) (width 1) (layer F.Cu) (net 60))
 (segment (start 159.695001 108.895001) (end 152.724999 108.895001) (width 1) (layer F.Cu) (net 60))
 (segment (start 154.615001 108.895001) (end 152.724999 108.895001) (width 1) (layer F.Cu) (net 60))
 (segment (start 152.724999 108.895001) (end 148.755001 108.895001) (width 1) (layer F.Cu) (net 60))
 (segment (start 148.755001 110.895001) (end 150.265001 110.895001) (width 0.25) (layer F.Cu) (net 62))
 (segment (start 161.29 113.03) (end 162.56 113.03) (width 1) (layer F.Cu) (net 62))
 (segment (start 148.755001 110.895001) (end 159.155001 110.895001) (width 1) (layer F.Cu) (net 62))
 (segment (start 159.155001 110.895001) (end 161.29 113.03) (width 1) (layer F.Cu) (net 62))
 (segment (start 133.555001 102.895001) (end 128.295001 102.895001) (width 1) (layer F.Cu) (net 63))
 (segment (start 128.295001 102.895001) (end 128.27 102.87) (width 1) (layer F.Cu) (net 63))
 (segment (start 128.295001 102.895001) (end 128.244999 102.895001) (width 1) (layer F.Cu) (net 63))
 (segment (start 163.83 96.52) (end 163.83 102.87) (width 1) (layer F.Cu) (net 58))
 (segment (start 164.48 103.52) (end 164.48 105.41) (width 1) (layer F.Cu) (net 58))
 (segment (start 163.83 102.87) (end 164.48 103.52) (width 1) (layer F.Cu) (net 58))
 (segment (start 161.074999 106.895001) (end 162.56 105.41) (width 1) (layer F.Cu) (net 58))
 (segment (start 153.835001 106.895001) (end 161.074999 106.895001) (width 1) (layer F.Cu) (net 58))
 (segment (start 162.56 105.41) (end 164.48 105.41) (width 1) (layer F.Cu) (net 58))
 (segment (start 153.835001 106.895001) (end 148.755001 106.895001) (width 1) (layer F.Cu) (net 58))
 (segment (start 133.555001 98.895001) (end 132.805001 98.895001) (width 1) (layer F.Cu) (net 59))
 (segment (start 132.805001 98.895001) (end 132.640002 99.06) (width 1) (layer F.Cu) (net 59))
 (segment (start 133.390002 99.06) (end 133.555001 98.895001) (width 1) (layer F.Cu) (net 59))
 (segment (start 133.555001 98.895001) (end 128.434999 98.895001) (width 1) (layer F.Cu) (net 59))
 (segment (start 126.059998 96.52) (end 128.434999 98.895001) (width 1) (layer F.Cu) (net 59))
 (segment (start 124.46 96.52) (end 126.059998 96.52) (width 1) (layer F.Cu) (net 59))
 (segment (start 124.46 88.9) (end 124.46 78.74) (width 1) (layer F.Cu) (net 9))
 (segment (start 123.19 77.47) (end 123.19 72.39) (width 1) (layer F.Cu) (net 9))
 (segment (start 124.46 78.74) (end 123.19 77.47) (width 1) (layer F.Cu) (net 9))
 (segment (start 132.99 100.33) (end 133.555001 100.895001) (width 1) (layer F.Cu) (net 55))
 (segment (start 129.54 100.33) (end 132.99 100.33) (width 1) (layer F.Cu) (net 55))
 (segment (start 136.155001 116.574999) (end 136.155001 114.395001) (width 1) (layer F.Cu) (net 54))
 (segment (start 134.62 118.11) (end 136.155001 116.574999) (width 1) (layer F.Cu) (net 54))
 (segment (start 138.155001 117.114999) (end 138.155001 114.395001) (width 1) (layer F.Cu) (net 53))
 (segment (start 137.16 118.11) (end 138.155001 117.114999) (width 1) (layer F.Cu) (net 53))
 (segment (start 140.155001 117.295001) (end 140.155001 114.395001) (width 1) (layer F.Cu) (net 52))
 (segment (start 140.97 118.11) (end 140.155001 117.295001) (width 1) (layer F.Cu) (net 52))
 (segment (start 142.24 114.48) (end 142.155001 114.395001) (width 1) (layer F.Cu) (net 51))
 (segment (start 142.155001 116.755001) (end 142.155001 114.395001) (width 1) (layer F.Cu) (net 51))
 (segment (start 143.51 118.11) (end 142.155001 116.755001) (width 1) (layer F.Cu) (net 51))
 (segment (start 144.155001 116.215001) (end 144.155001 114.395001) (width 1) (layer F.Cu) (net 50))
 (segment (start 146.05 118.11) (end 144.155001 116.215001) (width 1) (layer F.Cu) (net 50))
 (segment (start 148.59 118.11) (end 146.05 115.57) (width 1) (layer F.Cu) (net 49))
 (segment (start 146.155001 115.464999) (end 146.155001 114.395001) (width 1) (layer F.Cu) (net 49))
 (segment (start 146.05 115.57) (end 146.155001 115.464999) (width 1) (layer F.Cu) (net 49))
 (segment (start 132.8 104.14) (end 133.555001 104.895001) (width 1) (layer F.Cu) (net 48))
 (segment (start 129.54 104.14) (end 132.8 104.14) (width 1) (layer F.Cu) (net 48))
 (segment (start 133.34 106.68) (end 133.555001 106.895001) (width 1) (layer F.Cu) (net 47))
 (segment (start 129.54 106.68) (end 133.34 106.68) (width 1) (layer F.Cu) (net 47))
 (segment (start 133.230002 109.22) (end 133.555001 108.895001) (width 1) (layer F.Cu) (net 46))
 (segment (start 129.54 109.22) (end 133.230002 109.22) (width 1) (layer F.Cu) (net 46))
 (segment (start 130.404999 110.895001) (end 133.555001 110.895001) (width 1) (layer F.Cu) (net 45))
 (segment (start 129.54 111.76) (end 130.404999 110.895001) (width 1) (layer F.Cu) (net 45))
 (segment (start 149.27 105.41) (end 148.755001 104.895001) (width 1) (layer F.Cu) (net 44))
 (segment (start 152.4 105.41) (end 149.27 105.41) (width 1) (layer F.Cu) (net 44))
 (segment (start 148.780002 102.87) (end 148.755001 102.895001) (width 1) (layer F.Cu) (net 43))
 (segment (start 152.4 102.87) (end 148.780002 102.87) (width 1) (layer F.Cu) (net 43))
 (segment (start 159.865 83.975) (end 160.02 83.975) (width 1) (layer F.Cu) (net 2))
 (segment (start 160.02 82.55) (end 160.02 83.975) (width 1) (layer F.Cu) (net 2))
 (segment (start 150.564999 100.895001) (end 148.755001 100.895001) (width 1) (layer F.Cu) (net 2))
 (segment (start 155.644999 100.895001) (end 150.564999 100.895001) (width 1) (layer F.Cu) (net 2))
 (segment (start 158.75 97.79) (end 155.644999 100.895001) (width 1) (layer F.Cu) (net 2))
 (segment (start 158.75 86.36) (end 158.75 97.79) (width 1) (layer F.Cu) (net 2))
 (segment (start 160.02 83.975) (end 160.02 85.09) (width 1) (layer F.Cu) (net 2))
 (segment (start 160.02 85.09) (end 158.75 86.36) (width 1) (layer F.Cu) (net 2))
 (segment (start 151.294999 98.895001) (end 152.564999 98.895001) (width 1) (layer F.Cu) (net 1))
 (segment (start 148.755001 98.895001) (end 151.294999 98.895001) (width 1) (layer F.Cu) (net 1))
 (segment (start 152.564999 98.895001) (end 153.67 97.79) (width 1) (layer F.Cu) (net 1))
 (segment (start 154.94 96.52) (end 152.564999 98.895001) (width 1) (layer F.Cu) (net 1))
 (segment (start 154.94 82.55) (end 154.94 96.52) (width 1) (layer F.Cu) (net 1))
 (segment (start 124.46 100.33) (end 120.65 104.14) (width 1) (layer F.Cu) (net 59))
 (segment (start 124.46 96.52) (end 124.46 100.33) (width 1) (layer F.Cu) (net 59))
 (segment (start 125.73 104.14) (end 127 102.87) (width 1) (layer F.Cu) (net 63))
 (segment (start 127.025001 102.895001) (end 128.295001 102.895001) (width 1) (layer F.Cu) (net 63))
 (segment (start 127 102.87) (end 127.025001 102.895001) (width 1) (layer F.Cu) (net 63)))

